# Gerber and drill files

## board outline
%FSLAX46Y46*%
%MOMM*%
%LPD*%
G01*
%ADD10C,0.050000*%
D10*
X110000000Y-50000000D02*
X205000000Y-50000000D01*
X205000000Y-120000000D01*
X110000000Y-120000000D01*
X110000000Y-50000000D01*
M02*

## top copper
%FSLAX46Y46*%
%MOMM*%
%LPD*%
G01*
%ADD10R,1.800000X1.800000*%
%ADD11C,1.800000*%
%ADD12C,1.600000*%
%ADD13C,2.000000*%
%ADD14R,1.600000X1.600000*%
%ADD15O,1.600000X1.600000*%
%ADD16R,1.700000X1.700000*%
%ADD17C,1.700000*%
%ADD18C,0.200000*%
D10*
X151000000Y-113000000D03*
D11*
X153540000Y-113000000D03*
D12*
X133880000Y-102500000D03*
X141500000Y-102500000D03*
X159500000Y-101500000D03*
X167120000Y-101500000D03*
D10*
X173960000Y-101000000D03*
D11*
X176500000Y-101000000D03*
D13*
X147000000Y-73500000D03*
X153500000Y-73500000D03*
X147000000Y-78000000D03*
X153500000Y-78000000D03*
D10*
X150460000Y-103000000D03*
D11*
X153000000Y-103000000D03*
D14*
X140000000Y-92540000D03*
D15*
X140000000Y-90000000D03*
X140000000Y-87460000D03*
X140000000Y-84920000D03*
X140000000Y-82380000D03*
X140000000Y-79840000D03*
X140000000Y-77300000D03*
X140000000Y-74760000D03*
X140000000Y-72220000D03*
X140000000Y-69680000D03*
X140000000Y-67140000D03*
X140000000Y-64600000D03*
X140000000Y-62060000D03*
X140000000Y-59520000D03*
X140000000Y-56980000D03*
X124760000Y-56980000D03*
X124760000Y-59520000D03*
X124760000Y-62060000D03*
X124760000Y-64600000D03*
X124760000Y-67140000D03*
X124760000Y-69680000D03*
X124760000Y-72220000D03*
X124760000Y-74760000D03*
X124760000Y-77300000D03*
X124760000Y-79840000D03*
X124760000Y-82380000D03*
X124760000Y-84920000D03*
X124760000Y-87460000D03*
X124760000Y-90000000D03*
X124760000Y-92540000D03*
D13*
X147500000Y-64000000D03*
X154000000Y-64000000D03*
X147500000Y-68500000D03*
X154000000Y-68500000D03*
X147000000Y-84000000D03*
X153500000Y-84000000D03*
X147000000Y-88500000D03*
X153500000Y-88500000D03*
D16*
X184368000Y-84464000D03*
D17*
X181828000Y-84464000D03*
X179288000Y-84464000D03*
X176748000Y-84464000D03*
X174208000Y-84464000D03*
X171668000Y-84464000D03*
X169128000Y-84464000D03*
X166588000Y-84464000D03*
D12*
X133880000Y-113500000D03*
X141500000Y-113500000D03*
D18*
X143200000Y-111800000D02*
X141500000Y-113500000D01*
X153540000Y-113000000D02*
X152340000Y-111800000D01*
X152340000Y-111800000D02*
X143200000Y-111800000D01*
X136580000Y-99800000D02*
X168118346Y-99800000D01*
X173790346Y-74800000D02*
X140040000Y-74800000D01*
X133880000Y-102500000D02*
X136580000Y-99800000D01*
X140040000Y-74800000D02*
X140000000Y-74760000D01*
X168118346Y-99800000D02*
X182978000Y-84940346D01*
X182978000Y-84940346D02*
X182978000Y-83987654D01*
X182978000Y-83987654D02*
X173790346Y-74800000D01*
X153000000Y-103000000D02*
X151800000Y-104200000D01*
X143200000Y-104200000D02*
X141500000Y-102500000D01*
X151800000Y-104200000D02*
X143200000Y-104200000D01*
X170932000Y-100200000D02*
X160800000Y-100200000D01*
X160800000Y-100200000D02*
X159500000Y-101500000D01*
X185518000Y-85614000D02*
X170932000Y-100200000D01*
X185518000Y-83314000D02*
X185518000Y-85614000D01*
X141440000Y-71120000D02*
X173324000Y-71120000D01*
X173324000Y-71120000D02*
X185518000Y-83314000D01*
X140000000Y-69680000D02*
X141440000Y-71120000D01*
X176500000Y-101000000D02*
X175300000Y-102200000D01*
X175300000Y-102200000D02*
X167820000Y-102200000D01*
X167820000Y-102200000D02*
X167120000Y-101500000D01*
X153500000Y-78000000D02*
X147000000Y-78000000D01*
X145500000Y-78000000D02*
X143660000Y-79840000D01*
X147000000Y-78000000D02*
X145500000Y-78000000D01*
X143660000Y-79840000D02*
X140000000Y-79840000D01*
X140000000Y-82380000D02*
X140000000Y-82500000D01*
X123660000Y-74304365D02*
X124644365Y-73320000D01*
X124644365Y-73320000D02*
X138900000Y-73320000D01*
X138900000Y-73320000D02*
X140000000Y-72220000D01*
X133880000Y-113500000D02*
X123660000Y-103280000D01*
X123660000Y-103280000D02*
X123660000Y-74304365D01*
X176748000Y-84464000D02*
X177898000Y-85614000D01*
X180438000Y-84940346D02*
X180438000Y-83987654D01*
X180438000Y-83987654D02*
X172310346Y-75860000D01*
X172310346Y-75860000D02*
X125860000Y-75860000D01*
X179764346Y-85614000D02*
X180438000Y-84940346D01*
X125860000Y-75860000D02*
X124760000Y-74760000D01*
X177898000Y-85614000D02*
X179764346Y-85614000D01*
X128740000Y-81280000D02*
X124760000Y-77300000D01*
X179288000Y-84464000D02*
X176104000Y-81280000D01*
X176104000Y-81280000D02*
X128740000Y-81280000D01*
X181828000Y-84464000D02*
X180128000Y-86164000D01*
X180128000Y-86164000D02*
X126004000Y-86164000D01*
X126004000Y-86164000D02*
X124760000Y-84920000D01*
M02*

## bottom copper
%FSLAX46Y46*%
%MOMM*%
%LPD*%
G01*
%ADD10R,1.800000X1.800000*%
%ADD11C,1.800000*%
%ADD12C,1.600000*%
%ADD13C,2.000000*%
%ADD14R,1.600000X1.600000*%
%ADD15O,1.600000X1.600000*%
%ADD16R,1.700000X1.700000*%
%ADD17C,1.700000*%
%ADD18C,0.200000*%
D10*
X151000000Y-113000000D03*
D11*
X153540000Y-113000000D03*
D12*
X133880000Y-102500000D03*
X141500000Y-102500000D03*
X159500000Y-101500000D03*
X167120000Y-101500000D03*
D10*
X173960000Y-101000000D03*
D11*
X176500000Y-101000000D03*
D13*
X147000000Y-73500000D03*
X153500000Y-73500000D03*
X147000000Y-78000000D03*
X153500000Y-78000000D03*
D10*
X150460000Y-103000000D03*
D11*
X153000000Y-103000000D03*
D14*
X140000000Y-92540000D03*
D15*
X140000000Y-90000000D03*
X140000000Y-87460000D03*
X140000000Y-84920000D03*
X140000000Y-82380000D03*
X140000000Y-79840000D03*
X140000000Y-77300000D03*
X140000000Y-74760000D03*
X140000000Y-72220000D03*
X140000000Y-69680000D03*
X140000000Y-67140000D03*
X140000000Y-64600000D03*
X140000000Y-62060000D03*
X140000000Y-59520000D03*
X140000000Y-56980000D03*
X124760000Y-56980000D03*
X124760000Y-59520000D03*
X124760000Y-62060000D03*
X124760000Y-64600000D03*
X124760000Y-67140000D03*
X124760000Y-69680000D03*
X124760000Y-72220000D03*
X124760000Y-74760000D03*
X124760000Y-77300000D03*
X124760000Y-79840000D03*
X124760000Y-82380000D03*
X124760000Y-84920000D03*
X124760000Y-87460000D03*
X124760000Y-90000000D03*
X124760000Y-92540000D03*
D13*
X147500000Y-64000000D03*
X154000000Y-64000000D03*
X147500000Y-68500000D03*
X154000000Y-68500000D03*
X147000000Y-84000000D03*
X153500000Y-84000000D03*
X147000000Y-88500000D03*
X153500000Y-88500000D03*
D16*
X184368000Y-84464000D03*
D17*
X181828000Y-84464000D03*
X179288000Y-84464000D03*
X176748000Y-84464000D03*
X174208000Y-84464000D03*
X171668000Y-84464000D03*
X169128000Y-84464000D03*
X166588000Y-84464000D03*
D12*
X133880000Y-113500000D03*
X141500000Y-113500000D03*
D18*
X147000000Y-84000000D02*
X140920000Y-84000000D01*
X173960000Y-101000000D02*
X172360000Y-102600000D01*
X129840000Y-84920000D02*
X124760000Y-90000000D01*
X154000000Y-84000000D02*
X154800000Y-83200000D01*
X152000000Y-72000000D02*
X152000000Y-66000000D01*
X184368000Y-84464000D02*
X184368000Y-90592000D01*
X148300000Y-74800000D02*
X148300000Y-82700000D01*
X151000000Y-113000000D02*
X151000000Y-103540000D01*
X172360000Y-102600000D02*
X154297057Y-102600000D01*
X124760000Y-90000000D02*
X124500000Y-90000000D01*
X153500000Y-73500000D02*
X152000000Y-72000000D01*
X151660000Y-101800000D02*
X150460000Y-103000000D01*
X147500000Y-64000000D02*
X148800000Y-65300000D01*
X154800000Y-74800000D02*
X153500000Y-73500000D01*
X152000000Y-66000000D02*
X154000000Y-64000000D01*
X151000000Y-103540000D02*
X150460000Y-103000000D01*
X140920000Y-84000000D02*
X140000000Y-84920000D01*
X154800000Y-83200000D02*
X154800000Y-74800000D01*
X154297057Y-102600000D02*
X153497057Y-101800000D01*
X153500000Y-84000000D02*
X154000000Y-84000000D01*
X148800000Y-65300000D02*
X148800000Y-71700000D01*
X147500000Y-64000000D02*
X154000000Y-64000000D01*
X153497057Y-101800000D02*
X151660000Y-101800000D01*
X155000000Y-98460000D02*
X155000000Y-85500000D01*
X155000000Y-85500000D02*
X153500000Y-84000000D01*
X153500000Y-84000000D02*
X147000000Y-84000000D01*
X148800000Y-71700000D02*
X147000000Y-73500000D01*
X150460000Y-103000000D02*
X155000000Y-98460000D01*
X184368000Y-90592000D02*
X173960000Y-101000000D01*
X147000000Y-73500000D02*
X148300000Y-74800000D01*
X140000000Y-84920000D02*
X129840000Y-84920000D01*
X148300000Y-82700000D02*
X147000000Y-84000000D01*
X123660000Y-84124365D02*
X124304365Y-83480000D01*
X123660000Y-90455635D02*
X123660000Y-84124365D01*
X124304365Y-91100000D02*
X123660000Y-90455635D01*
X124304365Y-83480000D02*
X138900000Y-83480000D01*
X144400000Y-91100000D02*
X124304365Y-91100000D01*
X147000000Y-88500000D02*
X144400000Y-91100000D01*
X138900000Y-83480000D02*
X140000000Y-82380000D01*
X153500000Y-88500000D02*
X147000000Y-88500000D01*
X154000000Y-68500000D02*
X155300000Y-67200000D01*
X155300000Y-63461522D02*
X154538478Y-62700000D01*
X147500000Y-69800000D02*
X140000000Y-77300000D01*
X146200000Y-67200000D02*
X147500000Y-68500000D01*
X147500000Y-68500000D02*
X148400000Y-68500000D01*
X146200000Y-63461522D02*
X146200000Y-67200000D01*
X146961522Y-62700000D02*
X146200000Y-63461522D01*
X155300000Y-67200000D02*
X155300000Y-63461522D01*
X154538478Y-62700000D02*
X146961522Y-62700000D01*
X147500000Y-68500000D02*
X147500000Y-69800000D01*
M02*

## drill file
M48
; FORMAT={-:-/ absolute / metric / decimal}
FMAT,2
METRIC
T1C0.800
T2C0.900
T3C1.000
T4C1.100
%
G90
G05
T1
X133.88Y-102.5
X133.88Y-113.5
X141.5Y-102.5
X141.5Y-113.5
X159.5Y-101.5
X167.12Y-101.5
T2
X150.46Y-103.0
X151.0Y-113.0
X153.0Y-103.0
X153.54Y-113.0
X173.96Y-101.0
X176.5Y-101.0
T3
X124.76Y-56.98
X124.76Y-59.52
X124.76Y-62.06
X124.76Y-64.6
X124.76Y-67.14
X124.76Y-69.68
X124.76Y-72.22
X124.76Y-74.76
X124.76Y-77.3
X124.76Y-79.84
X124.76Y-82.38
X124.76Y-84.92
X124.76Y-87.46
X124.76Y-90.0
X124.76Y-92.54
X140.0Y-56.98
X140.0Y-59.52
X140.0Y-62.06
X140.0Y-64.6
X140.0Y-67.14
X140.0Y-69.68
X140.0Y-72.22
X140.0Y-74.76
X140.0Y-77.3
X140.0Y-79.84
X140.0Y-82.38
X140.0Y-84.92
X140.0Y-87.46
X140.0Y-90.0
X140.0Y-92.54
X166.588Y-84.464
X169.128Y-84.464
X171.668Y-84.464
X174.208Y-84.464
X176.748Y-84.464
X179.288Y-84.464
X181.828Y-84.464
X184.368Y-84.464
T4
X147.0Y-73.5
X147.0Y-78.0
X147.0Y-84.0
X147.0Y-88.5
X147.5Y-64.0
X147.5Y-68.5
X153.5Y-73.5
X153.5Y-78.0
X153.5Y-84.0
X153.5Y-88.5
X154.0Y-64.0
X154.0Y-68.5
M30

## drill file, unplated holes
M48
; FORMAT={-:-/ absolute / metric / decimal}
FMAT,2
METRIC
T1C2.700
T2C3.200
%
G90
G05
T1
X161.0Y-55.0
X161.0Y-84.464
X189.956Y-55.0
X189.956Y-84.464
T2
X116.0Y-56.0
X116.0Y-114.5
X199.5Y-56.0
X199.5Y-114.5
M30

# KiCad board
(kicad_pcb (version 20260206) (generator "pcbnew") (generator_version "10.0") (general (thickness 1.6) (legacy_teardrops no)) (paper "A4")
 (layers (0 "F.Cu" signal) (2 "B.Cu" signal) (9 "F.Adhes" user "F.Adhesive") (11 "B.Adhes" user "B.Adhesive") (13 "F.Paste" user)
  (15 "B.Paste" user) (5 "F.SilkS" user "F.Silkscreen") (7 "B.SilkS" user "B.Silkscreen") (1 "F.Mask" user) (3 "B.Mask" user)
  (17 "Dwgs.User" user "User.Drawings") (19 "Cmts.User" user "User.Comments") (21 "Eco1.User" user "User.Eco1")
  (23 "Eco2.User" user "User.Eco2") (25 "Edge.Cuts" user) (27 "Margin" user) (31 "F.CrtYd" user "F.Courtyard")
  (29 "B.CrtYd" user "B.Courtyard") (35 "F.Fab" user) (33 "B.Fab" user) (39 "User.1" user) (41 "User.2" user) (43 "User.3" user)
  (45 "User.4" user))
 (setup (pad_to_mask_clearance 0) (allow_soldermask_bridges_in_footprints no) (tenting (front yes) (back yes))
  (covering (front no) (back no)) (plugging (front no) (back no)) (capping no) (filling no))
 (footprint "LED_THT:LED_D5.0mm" (layer "F.Cu") (at 151 113)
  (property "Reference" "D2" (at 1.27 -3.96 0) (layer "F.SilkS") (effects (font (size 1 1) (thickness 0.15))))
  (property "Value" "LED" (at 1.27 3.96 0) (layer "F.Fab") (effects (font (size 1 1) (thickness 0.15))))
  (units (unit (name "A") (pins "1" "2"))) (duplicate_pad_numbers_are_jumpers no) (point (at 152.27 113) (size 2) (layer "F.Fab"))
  (pad "1" thru_hole rect (at 0 0) (size 1.8 1.8) (drill 0.9) (layers "*.Cu" "*.Mask") (remove_unused_layers no) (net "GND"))
  (pad "2" thru_hole circle (at 2.54 0) (size 1.8 1.8) (drill 0.9) (layers "*.Cu" "*.Mask") (remove_unused_layers no) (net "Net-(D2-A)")))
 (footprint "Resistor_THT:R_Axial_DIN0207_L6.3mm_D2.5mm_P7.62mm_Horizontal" (layer "F.Cu") (at 133.88 102.5)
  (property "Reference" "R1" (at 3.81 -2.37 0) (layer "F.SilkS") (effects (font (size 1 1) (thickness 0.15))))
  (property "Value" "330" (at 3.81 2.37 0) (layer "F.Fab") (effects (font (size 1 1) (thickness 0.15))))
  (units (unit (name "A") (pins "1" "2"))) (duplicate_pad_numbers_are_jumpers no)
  (pad "1" thru_hole circle (at 0 0) (size 1.6 1.6) (drill 0.8) (layers "*.Cu" "*.Mask") (remove_unused_layers no) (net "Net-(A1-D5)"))
  (pad "2" thru_hole circle (at 7.62 0) (size 1.6 1.6) (drill 0.8) (layers "*.Cu" "*.Mask") (remove_unused_layers no) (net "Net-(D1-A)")))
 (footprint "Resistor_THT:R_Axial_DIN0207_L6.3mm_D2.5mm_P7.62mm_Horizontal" (layer "F.Cu") (at 159.5 101.5)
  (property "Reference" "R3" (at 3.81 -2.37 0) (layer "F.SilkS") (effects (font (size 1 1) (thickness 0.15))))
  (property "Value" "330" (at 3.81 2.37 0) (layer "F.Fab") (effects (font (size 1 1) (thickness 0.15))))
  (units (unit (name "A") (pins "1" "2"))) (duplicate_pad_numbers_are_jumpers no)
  (pad "1" thru_hole circle (at 0 0) (size 1.6 1.6) (drill 0.8) (layers "*.Cu" "*.Mask") (remove_unused_layers no) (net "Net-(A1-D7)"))
  (pad "2" thru_hole circle (at 7.62 0) (size 1.6 1.6) (drill 0.8) (layers "*.Cu" "*.Mask") (remove_unused_layers no) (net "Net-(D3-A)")))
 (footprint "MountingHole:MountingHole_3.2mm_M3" (layer "F.Cu") (at 199.5 114.5)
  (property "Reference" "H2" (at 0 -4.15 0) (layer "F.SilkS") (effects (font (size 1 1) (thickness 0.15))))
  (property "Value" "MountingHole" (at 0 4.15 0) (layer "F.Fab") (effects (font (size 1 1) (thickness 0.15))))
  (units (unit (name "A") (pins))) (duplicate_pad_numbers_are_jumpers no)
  (pad "" np_thru_hole circle (at 0 0) (size 3.2 3.2) (drill 3.2) (layers "*.Cu" "*.Mask")))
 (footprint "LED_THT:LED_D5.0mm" (layer "F.Cu") (at 173.96 101)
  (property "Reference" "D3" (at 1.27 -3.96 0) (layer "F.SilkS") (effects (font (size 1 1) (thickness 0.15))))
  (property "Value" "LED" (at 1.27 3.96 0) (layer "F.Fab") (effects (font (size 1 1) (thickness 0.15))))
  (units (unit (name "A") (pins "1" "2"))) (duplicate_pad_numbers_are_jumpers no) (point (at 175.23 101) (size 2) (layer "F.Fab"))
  (pad "1" thru_hole rect (at 0 0) (size 1.8 1.8) (drill 0.9) (layers "*.Cu" "*.Mask") (remove_unused_layers no) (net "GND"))
  (pad "2" thru_hole circle (at 2.54 0) (size 1.8 1.8) (drill 0.9) (layers "*.Cu" "*.Mask") (remove_unused_layers no) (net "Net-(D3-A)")))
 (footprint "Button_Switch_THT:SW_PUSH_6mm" (layer "F.Cu") (at 147 73.5)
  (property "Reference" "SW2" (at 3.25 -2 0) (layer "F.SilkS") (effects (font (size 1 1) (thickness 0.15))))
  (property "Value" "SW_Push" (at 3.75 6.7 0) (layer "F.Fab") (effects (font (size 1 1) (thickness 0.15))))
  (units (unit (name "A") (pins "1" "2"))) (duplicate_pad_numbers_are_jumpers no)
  (pad "1" thru_hole circle (at 0 0 90) (size 2 2) (drill 1.1) (layers "*.Cu" "*.Mask") (remove_unused_layers no) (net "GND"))
  (pad "1" thru_hole circle (at 6.5 0 90) (size 2 2) (drill 1.1) (layers "*.Cu" "*.Mask") (remove_unused_layers no) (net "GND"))
  (pad "2" thru_hole circle (at 0 4.5 90) (size 2 2) (drill 1.1) (layers "*.Cu" "*.Mask") (remove_unused_layers no) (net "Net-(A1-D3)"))
  (pad "2" thru_hole circle (at 6.5 4.5 90) (size 2 2) (drill 1.1) (layers "*.Cu" "*.Mask") (remove_unused_layers no) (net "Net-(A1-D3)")))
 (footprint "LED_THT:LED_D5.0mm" (layer "F.Cu") (at 150.46 103)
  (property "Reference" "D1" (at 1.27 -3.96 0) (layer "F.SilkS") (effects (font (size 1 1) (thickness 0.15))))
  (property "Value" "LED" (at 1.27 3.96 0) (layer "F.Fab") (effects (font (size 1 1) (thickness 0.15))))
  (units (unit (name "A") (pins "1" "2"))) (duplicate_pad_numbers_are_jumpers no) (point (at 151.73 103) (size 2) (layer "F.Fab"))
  (pad "1" thru_hole rect (at 0 0) (size 1.8 1.8) (drill 0.9) (layers "*.Cu" "*.Mask") (remove_unused_layers no) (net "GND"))
  (pad "2" thru_hole circle (at 2.54 0) (size 1.8 1.8) (drill 0.9) (layers "*.Cu" "*.Mask") (remove_unused_layers no) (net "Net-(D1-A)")))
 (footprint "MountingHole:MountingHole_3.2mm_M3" (layer "F.Cu") (at 199.5 56)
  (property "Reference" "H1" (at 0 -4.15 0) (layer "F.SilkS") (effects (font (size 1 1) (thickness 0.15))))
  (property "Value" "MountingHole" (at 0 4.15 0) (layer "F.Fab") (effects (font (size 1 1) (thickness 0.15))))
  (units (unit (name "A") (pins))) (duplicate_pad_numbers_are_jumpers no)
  (pad "" np_thru_hole circle (at 0 0) (size 3.2 3.2) (drill 3.2) (layers "*.Cu" "*.Mask")))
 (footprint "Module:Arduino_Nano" (layer "F.Cu") (at 140 92.54 180)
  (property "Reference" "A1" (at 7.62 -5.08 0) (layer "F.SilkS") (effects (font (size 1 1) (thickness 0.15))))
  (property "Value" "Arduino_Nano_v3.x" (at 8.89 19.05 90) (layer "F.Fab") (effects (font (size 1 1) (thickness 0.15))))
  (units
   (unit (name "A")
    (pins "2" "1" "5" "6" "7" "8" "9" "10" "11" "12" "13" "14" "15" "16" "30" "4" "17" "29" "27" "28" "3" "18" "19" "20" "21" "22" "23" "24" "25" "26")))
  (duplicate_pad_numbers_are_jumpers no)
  (pad "1" thru_hole rect (at 0 0 180) (size 1.6 1.6) (drill 1) (layers "*.Cu" "*.Mask") (remove_unused_layers no)
   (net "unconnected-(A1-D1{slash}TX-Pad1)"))
  (pad "2" thru_hole oval (at 0 2.54 180) (size 1.6 1.6) (drill 1) (layers "*.Cu" "*.Mask") (remove_unused_layers no)
   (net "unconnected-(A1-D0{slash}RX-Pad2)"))
  (pad "3" thru_hole oval (at 0 5.08 180) (size 1.6 1.6) (drill 1) (layers "*.Cu" "*.Mask") (remove_unused_layers no)
   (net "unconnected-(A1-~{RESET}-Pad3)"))
  (pad "4" thru_hole oval (at 0 7.62 180) (size 1.6 1.6) (drill 1) (layers "*.Cu" "*.Mask") (remove_unused_layers no) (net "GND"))
  (pad "5" thru_hole oval (at 0 10.16 180) (size 1.6 1.6) (drill 1) (layers "*.Cu" "*.Mask") (remove_unused_layers no) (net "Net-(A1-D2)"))
  (pad "6" thru_hole oval (at 0 12.7 180) (size 1.6 1.6) (drill 1) (layers "*.Cu" "*.Mask") (remove_unused_layers no) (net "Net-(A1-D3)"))
  (pad "7" thru_hole oval (at 0 15.24 180) (size 1.6 1.6) (drill 1) (layers "*.Cu" "*.Mask") (remove_unused_layers no) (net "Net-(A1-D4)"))
  (pad "8" thru_hole oval (at 0 17.78 180) (size 1.6 1.6) (drill 1) (layers "*.Cu" "*.Mask") (remove_unused_layers no) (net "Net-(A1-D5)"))
  (pad "9" thru_hole oval (at 0 20.32 180) (size 1.6 1.6) (drill 1) (layers "*.Cu" "*.Mask") (remove_unused_layers no) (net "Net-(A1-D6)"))
  (pad "10" thru_hole oval (at 0 22.86 180) (size 1.6 1.6) (drill 1) (layers "*.Cu" "*.Mask") (remove_unused_layers no) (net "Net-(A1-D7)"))
  (pad "11" thru_hole oval (at 0 25.4 180) (size 1.6 1.6) (drill 1) (layers "*.Cu" "*.Mask") (remove_unused_layers no)
   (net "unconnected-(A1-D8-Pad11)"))
  (pad "12" thru_hole oval (at 0 27.94 180) (size 1.6 1.6) (drill 1) (layers "*.Cu" "*.Mask") (remove_unused_layers no)
   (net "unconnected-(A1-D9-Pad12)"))
  (pad "13" thru_hole oval (at 0 30.48 180) (size 1.6 1.6) (drill 1) (layers "*.Cu" "*.Mask") (remove_unused_layers no)
   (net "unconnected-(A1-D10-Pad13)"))
  (pad "14" thru_hole oval (at 0 33.02 180) (size 1.6 1.6) (drill 1) (layers "*.Cu" "*.Mask") (remove_unused_layers no)
   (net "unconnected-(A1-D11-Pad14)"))
  (pad "15" thru_hole oval (at 0 35.56 180) (size 1.6 1.6) (drill 1) (layers "*.Cu" "*.Mask") (remove_unused_layers no)
   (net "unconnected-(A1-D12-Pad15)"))
  (pad "16" thru_hole oval (at 15.24 35.56 180) (size 1.6 1.6) (drill 1) (layers "*.Cu" "*.Mask") (remove_unused_layers no)
   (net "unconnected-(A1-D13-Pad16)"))
  (pad "17" thru_hole oval (at 15.24 33.02 180) (size 1.6 1.6) (drill 1) (layers "*.Cu" "*.Mask") (remove_unused_layers no)
   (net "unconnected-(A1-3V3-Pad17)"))
  (pad "18" thru_hole oval (at 15.24 30.48 180) (size 1.6 1.6) (drill 1) (layers "*.Cu" "*.Mask") (remove_unused_layers no)
   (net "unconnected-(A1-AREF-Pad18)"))
  (pad "19" thru_hole oval (at 15.24 27.94 180) (size 1.6 1.6) (drill 1) (layers "*.Cu" "*.Mask") (remove_unused_layers no)
   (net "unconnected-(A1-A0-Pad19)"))
  (pad "20" thru_hole oval (at 15.24 25.4 180) (size 1.6 1.6) (drill 1) (layers "*.Cu" "*.Mask") (remove_unused_layers no)
   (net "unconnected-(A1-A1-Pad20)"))
  (pad "21" thru_hole oval (at 15.24 22.86 180) (size 1.6 1.6) (drill 1) (layers "*.Cu" "*.Mask") (remove_unused_layers no)
   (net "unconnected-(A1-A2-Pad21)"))
  (pad "22" thru_hole oval (at 15.24 20.32 180) (size 1.6 1.6) (drill 1) (layers "*.Cu" "*.Mask") (remove_unused_layers no)
   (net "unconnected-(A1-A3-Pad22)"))
  (pad "23" thru_hole oval (at 15.24 17.78 180) (size 1.6 1.6) (drill 1) (layers "*.Cu" "*.Mask") (remove_unused_layers no) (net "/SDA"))
  (pad "24" thru_hole oval (at 15.24 15.24 180) (size 1.6 1.6) (drill 1) (layers "*.Cu" "*.Mask") (remove_unused_layers no) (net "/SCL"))
  (pad "25" thru_hole oval (at 15.24 12.7 180) (size 1.6 1.6) (drill 1) (layers "*.Cu" "*.Mask") (remove_unused_layers no)
   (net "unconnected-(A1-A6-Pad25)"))
  (pad "26" thru_hole oval (at 15.24 10.16 180) (size 1.6 1.6) (drill 1) (layers "*.Cu" "*.Mask") (remove_unused_layers no)
   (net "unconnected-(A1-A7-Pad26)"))
  (pad "27" thru_hole oval (at 15.24 7.62 180) (size 1.6 1.6) (drill 1) (layers "*.Cu" "*.Mask") (remove_unused_layers no) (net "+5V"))
  (pad "28" thru_hole oval (at 15.24 5.08 180) (size 1.6 1.6) (drill 1) (layers "*.Cu" "*.Mask") (remove_unused_layers no)
   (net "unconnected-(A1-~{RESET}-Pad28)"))
  (pad "29" thru_hole oval (at 15.24 2.54 180) (size 1.6 1.6) (drill 1) (layers "*.Cu" "*.Mask") (remove_unused_layers no) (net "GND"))
  (pad "30" thru_hole oval (at 15.24 0 180) (size 1.6 1.6) (drill 1) (layers "*.Cu" "*.Mask") (remove_unused_layers no)
   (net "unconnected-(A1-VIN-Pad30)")))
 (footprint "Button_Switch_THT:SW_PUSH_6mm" (layer "F.Cu") (at 147.5 64)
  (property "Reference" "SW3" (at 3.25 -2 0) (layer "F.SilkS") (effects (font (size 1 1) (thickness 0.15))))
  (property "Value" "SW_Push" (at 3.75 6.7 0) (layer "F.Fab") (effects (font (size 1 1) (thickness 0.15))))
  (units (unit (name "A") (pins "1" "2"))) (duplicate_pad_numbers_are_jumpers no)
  (pad "1" thru_hole circle (at 0 0 90) (size 2 2) (drill 1.1) (layers "*.Cu" "*.Mask") (remove_unused_layers no) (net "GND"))
  (pad "1" thru_hole circle (at 6.5 0 90) (size 2 2) (drill 1.1) (layers "*.Cu" "*.Mask") (remove_unused_layers no) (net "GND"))
  (pad "2" thru_hole circle (at 0 4.5 90) (size 2 2) (drill 1.1) (layers "*.Cu" "*.Mask") (remove_unused_layers no) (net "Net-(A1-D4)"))
  (pad "2" thru_hole circle (at 6.5 4.5 90) (size 2 2) (drill 1.1) (layers "*.Cu" "*.Mask") (remove_unused_layers no) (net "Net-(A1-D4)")))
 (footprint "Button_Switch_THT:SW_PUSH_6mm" (layer "F.Cu") (at 147 84)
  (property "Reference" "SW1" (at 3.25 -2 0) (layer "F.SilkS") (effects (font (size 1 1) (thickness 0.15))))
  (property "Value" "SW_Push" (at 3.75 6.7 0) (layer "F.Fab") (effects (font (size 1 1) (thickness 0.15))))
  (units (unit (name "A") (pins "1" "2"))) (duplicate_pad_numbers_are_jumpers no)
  (pad "1" thru_hole circle (at 0 0 90) (size 2 2) (drill 1.1) (layers "*.Cu" "*.Mask") (remove_unused_layers no) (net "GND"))
  (pad "1" thru_hole circle (at 6.5 0 90) (size 2 2) (drill 1.1) (layers "*.Cu" "*.Mask") (remove_unused_layers no) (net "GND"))
  (pad "2" thru_hole circle (at 0 4.5 90) (size 2 2) (drill 1.1) (layers "*.Cu" "*.Mask") (remove_unused_layers no) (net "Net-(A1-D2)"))
  (pad "2" thru_hole circle (at 6.5 4.5 90) (size 2 2) (drill 1.1) (layers "*.Cu" "*.Mask") (remove_unused_layers no) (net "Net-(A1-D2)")))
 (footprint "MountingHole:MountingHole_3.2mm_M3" (layer "F.Cu") (at 116 56)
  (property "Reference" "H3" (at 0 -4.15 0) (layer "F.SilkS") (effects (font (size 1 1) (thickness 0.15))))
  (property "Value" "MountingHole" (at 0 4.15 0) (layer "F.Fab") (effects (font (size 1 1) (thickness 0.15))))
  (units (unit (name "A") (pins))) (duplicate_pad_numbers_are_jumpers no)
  (pad "" np_thru_hole circle (at 0 0) (size 3.2 3.2) (drill 3.2) (layers "*.Cu" "*.Mask")))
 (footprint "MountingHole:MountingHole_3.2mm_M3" (layer "F.Cu") (at 116 114.5)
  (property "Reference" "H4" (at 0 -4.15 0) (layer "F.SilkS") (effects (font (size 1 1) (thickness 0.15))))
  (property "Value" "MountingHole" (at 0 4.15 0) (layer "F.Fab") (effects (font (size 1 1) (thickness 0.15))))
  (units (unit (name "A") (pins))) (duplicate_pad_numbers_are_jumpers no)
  (pad "" np_thru_hole circle (at 0 0) (size 3.2 3.2) (drill 3.2) (layers "*.Cu" "*.Mask")))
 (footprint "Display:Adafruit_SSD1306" (layer "F.Cu") (at 184.368 84.464 180)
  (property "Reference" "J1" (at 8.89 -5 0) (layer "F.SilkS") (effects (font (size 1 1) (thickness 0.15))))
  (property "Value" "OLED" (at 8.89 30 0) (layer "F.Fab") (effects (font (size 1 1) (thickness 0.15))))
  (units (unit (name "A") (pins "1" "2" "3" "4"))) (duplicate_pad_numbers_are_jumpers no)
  (pad "" np_thru_hole circle (at -5.588 0 180) (size 2.7 2.7) (drill 2.7) (layers "*.Cu" "*.Mask"))
  (pad "" np_thru_hole circle (at -5.588 29.464 180) (size 2.7 2.7) (drill 2.7) (layers "*.Cu" "*.Mask"))
  (pad "" np_thru_hole circle (at 23.368 0 180) (size 2.7 2.7) (drill 2.7) (layers "*.Cu" "*.Mask"))
  (pad "" np_thru_hole circle (at 23.368 29.464 180) (size 2.7 2.7) (drill 2.7) (layers "*.Cu" "*.Mask"))
  (pad "1" thru_hole rect (at 0 0 180) (size 1.7 1.7) (drill 1) (layers "*.Cu" "*.Mask") (remove_unused_layers no) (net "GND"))
  (pad "2" thru_hole circle (at 2.54 0 180) (size 1.7 1.7) (drill 1) (layers "*.Cu" "*.Mask") (remove_unused_layers no) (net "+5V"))
  (pad "3" thru_hole circle (at 5.08 0 180) (size 1.7 1.7) (drill 1) (layers "*.Cu" "*.Mask") (remove_unused_layers no) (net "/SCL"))
  (pad "4" thru_hole circle (at 7.62 0 180) (size 1.7 1.7) (drill 1) (layers "*.Cu" "*.Mask") (remove_unused_layers no) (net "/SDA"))
  (pad "5" thru_hole circle (at 10.16 0 180) (size 1.7 1.7) (drill 1) (layers "*.Cu" "*.Mask") (remove_unused_layers no))
  (pad "6" thru_hole circle (at 12.7 0 180) (size 1.7 1.7) (drill 1) (layers "*.Cu" "*.Mask") (remove_unused_layers no))
  (pad "7" thru_hole circle (at 15.24 0 180) (size 1.7 1.7) (drill 1) (layers "*.Cu" "*.Mask") (remove_unused_layers no))
  (pad "8" thru_hole circle (at 17.78 0 180) (size 1.7 1.7) (drill 1) (layers "*.Cu" "*.Mask") (remove_unused_layers no)))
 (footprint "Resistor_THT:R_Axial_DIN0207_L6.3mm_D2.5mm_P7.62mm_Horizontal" (layer "F.Cu") (at 133.88 113.5)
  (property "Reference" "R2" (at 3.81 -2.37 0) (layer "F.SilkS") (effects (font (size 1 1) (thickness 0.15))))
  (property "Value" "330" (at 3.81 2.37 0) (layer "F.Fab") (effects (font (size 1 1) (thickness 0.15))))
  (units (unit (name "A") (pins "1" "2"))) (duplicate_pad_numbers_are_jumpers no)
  (pad "1" thru_hole circle (at 0 0) (size 1.6 1.6) (drill 0.8) (layers "*.Cu" "*.Mask") (remove_unused_layers no) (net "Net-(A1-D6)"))
  (pad "2" thru_hole circle (at 7.62 0) (size 1.6 1.6) (drill 0.8) (layers "*.Cu" "*.Mask") (remove_unused_layers no) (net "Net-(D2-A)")))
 (gr_rect (start 110 50) (end 205 120) (stroke (width 0.05) (type default)) (fill no) (layer "Edge.Cuts"))
 (segment (start 147 84) (end 140.92 84) (width 0.2) (layer "B.Cu") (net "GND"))
 (segment (start 173.96 101) (end 172.36 102.6) (width 0.2) (layer "B.Cu") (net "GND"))
 (segment (start 129.84 84.92) (end 124.76 90) (width 0.2) (layer "B.Cu") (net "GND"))
 (segment (start 154 84) (end 154.8 83.2) (width 0.2) (layer "B.Cu") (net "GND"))
 (segment (start 152 72) (end 152 66) (width 0.2) (layer "B.Cu") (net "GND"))
 (segment (start 184.368 84.464) (end 184.368 90.592) (width 0.2) (layer "B.Cu") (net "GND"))
 (segment (start 148.3 74.8) (end 148.3 82.7) (width 0.2) (layer "B.Cu") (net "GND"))
 (segment (start 151 113) (end 151 103.54) (width 0.2) (layer "B.Cu") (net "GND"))
 (segment (start 172.36 102.6) (end 154.297057 102.6) (width 0.2) (layer "B.Cu") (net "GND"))
 (segment (start 124.76 90) (end 124.5 90) (width 0.2) (layer "B.Cu") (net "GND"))
 (segment (start 153.5 73.5) (end 152 72) (width 0.2) (layer "B.Cu") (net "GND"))
 (segment (start 151.66 101.8) (end 150.46 103) (width 0.2) (layer "B.Cu") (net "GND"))
 (segment (start 147.5 64) (end 148.8 65.3) (width 0.2) (layer "B.Cu") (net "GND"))
 (segment (start 154.8 74.8) (end 153.5 73.5) (width 0.2) (layer "B.Cu") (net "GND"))
 (segment (start 152 66) (end 154 64) (width 0.2) (layer "B.Cu") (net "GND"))
 (segment (start 151 103.54) (end 150.46 103) (width 0.2) (layer "B.Cu") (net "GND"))
 (segment (start 140.92 84) (end 140 84.92) (width 0.2) (layer "B.Cu") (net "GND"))
 (segment (start 154.8 83.2) (end 154.8 74.8) (width 0.2) (layer "B.Cu") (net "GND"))
 (segment (start 154.297057 102.6) (end 153.497057 101.8) (width 0.2) (layer "B.Cu") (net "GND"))
 (segment (start 153.5 84) (end 154 84) (width 0.2) (layer "B.Cu") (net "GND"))
 (segment (start 148.8 65.3) (end 148.8 71.7) (width 0.2) (layer "B.Cu") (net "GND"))
 (segment (start 147.5 64) (end 154 64) (width 0.2) (layer "B.Cu") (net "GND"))
 (segment (start 153.497057 101.8) (end 151.66 101.8) (width 0.2) (layer "B.Cu") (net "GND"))
 (segment (start 155 98.46) (end 155 85.5) (width 0.2) (layer "B.Cu") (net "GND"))
 (segment (start 155 85.5) (end 153.5 84) (width 0.2) (layer "B.Cu") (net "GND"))
 (segment (start 153.5 84) (end 147 84) (width 0.2) (layer "B.Cu") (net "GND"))
 (segment (start 148.8 71.7) (end 147 73.5) (width 0.2) (layer "B.Cu") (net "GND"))
 (segment (start 150.46 103) (end 155 98.46) (width 0.2) (layer "B.Cu") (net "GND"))
 (segment (start 184.368 90.592) (end 173.96 101) (width 0.2) (layer "B.Cu") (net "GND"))
 (segment (start 147 73.5) (end 148.3 74.8) (width 0.2) (layer "B.Cu") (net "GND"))
 (segment (start 140 84.92) (end 129.84 84.92) (width 0.2) (layer "B.Cu") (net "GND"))
 (segment (start 148.3 82.7) (end 147 84) (width 0.2) (layer "B.Cu") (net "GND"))
 (segment (start 143.2 111.8) (end 141.5 113.5) (width 0.2) (layer "F.Cu") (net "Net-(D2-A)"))
 (segment (start 153.54 113) (end 152.34 111.8) (width 0.2) (layer "F.Cu") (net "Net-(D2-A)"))
 (segment (start 152.34 111.8) (end 143.2 111.8) (width 0.2) (layer "F.Cu") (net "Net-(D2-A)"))
 (segment (start 136.58 99.8) (end 168.118346 99.8) (width 0.2) (layer "F.Cu") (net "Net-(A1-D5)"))
 (segment (start 173.790346 74.8) (end 140.04 74.8) (width 0.2) (layer "F.Cu") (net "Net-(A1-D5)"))
 (segment (start 133.88 102.5) (end 136.58 99.8) (width 0.2) (layer "F.Cu") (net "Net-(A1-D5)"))
 (segment (start 140.04 74.8) (end 140 74.76) (width 0.2) (layer "F.Cu") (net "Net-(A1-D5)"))
 (segment (start 168.118346 99.8) (end 182.978 84.940346) (width 0.2) (layer "F.Cu") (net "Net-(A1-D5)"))
 (segment (start 182.978 84.940346) (end 182.978 83.987654) (width 0.2) (layer "F.Cu") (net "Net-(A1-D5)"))
 (segment (start 182.978 83.987654) (end 173.790346 74.8) (width 0.2) (layer "F.Cu") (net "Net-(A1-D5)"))
 (segment (start 153 103) (end 151.8 104.2) (width 0.2) (layer "F.Cu") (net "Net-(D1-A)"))
 (segment (start 143.2 104.2) (end 141.5 102.5) (width 0.2) (layer "F.Cu") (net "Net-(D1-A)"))
 (segment (start 151.8 104.2) (end 143.2 104.2) (width 0.2) (layer "F.Cu") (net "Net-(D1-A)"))
 (segment (start 170.932 100.2) (end 160.8 100.2) (width 0.2) (layer "F.Cu") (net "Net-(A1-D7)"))
 (segment (start 160.8 100.2) (end 159.5 101.5) (width 0.2) (layer "F.Cu") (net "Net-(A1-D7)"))
 (segment (start 185.518 85.614) (end 170.932 100.2) (width 0.2) (layer "F.Cu") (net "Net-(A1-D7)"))
 (segment (start 185.518 83.314) (end 185.518 85.614) (width 0.2) (layer "F.Cu") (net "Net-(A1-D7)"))
 (segment (start 141.44 71.12) (end 173.324 71.12) (width 0.2) (layer "F.Cu") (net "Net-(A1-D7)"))
 (segment (start 173.324 71.12) (end 185.518 83.314) (width 0.2) (layer "F.Cu") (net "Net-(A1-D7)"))
 (segment (start 140 69.68) (end 141.44 71.12) (width 0.2) (layer "F.Cu") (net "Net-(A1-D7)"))
 (segment (start 176.5 101) (end 175.3 102.2) (width 0.2) (layer "F.Cu") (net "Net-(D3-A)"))
 (segment (start 175.3 102.2) (end 167.82 102.2) (width 0.2) (layer "F.Cu") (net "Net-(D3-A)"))
 (segment (start 167.82 102.2) (end 167.12 101.5) (width 0.2) (layer "F.Cu") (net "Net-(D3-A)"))
 (segment (start 153.5 78) (end 147 78) (width 0.2) (layer "F.Cu") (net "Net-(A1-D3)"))
 (segment (start 145.5 78) (end 143.66 79.84) (width 0.2) (layer "F.Cu") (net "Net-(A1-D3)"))
 (segment (start 147 78) (end 145.5 78) (width 0.2) (layer "F.Cu") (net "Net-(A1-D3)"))
 (segment (start 143.66 79.84) (end 140 79.84) (width 0.2) (layer "F.Cu") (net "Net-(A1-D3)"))
 (segment (start 140 82.38) (end 140 82.5) (width 0.2) (layer "F.Cu") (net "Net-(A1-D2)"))
 (segment (start 123.66 84.124365) (end 124.304365 83.48) (width 0.2) (layer "B.Cu") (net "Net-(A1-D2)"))
 (segment (start 123.66 90.455635) (end 123.66 84.124365) (width 0.2) (layer "B.Cu") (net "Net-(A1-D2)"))
 (segment (start 124.304365 91.1) (end 123.66 90.455635) (width 0.2) (layer "B.Cu") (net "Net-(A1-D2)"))
 (segment (start 124.304365 83.48) (end 138.9 83.48) (width 0.2) (layer "B.Cu") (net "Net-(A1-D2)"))
 (segment (start 144.4 91.1) (end 124.304365 91.1) (width 0.2) (layer "B.Cu") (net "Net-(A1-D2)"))
 (segment (start 147 88.5) (end 144.4 91.1) (width 0.2) (layer "B.Cu") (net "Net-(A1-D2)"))
 (segment (start 138.9 83.48) (end 140 82.38) (width 0.2) (layer "B.Cu") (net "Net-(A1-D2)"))
 (segment (start 153.5 88.5) (end 147 88.5) (width 0.2) (layer "B.Cu") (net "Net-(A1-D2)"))
 (segment (start 154 68.5) (end 155.3 67.2) (width 0.2) (layer "B.Cu") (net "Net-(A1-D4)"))
 (segment (start 155.3 63.461522) (end 154.538478 62.7) (width 0.2) (layer "B.Cu") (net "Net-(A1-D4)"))
 (segment (start 147.5 69.8) (end 140 77.3) (width 0.2) (layer "B.Cu") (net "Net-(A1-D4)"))
 (segment (start 146.2 67.2) (end 147.5 68.5) (width 0.2) (layer "B.Cu") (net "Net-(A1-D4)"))
 (segment (start 147.5 68.5) (end 148.4 68.5) (width 0.2) (layer "B.Cu") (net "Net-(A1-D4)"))
 (segment (start 146.2 63.461522) (end 146.2 67.2) (width 0.2) (layer "B.Cu") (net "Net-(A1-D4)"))
 (segment (start 146.961522 62.7) (end 146.2 63.461522) (width 0.2) (layer "B.Cu") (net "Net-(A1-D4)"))
 (segment (start 155.3 67.2) (end 155.3 63.461522) (width 0.2) (layer "B.Cu") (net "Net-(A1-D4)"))
 (segment (start 154.538478 62.7) (end 146.961522 62.7) (width 0.2) (layer "B.Cu") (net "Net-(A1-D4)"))
 (segment (start 147.5 68.5) (end 147.5 69.8) (width 0.2) (layer "B.Cu") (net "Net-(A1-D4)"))
 (segment (start 123.66 74.304365) (end 124.644365 73.32) (width 0.2) (layer "F.Cu") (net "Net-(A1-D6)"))
 (segment (start 124.644365 73.32) (end 138.9 73.32) (width 0.2) (layer "F.Cu") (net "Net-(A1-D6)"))
 (segment (start 138.9 73.32) (end 140 72.22) (width 0.2) (layer "F.Cu") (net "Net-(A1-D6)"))
 (segment (start 133.88 113.5) (end 123.66 103.28) (width 0.2) (layer "F.Cu") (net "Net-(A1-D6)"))
 (segment (start 123.66 103.28) (end 123.66 74.304365) (width 0.2) (layer "F.Cu") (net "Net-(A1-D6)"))
 (segment (start 176.748 84.464) (end 177.898 85.614) (width 0.2) (layer "F.Cu") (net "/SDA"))
 (segment (start 180.438 84.940346) (end 180.438 83.987654) (width 0.2) (layer "F.Cu") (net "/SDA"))
 (segment (start 180.438 83.987654) (end 172.310346 75.86) (width 0.2) (layer "F.Cu") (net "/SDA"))
 (segment (start 172.310346 75.86) (end 125.86 75.86) (width 0.2) (layer "F.Cu") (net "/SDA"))
 (segment (start 179.764346 85.614) (end 180.438 84.940346) (width 0.2) (layer "F.Cu") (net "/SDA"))
 (segment (start 125.86 75.86) (end 124.76 74.76) (width 0.2) (layer "F.Cu") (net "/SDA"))
 (segment (start 177.898 85.614) (end 179.764346 85.614) (width 0.2) (layer "F.Cu") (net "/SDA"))
 (segment (start 128.74 81.28) (end 124.76 77.3) (width 0.2) (layer "F.Cu") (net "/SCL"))
 (segment (start 179.288 84.464) (end 176.104 81.28) (width 0.2) (layer "F.Cu") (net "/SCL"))
 (segment (start 176.104 81.28) (end 128.74 81.28) (width 0.2) (layer "F.Cu") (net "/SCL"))
 (segment (start 181.828 84.464) (end 180.128 86.164) (width 0.2) (layer "F.Cu") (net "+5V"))
 (segment (start 180.128 86.164) (end 126.004 86.164) (width 0.2) (layer "F.Cu") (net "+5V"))
 (segment (start 126.004 86.164) (end 124.76 84.92) (width 0.2) (layer "F.Cu") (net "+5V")))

